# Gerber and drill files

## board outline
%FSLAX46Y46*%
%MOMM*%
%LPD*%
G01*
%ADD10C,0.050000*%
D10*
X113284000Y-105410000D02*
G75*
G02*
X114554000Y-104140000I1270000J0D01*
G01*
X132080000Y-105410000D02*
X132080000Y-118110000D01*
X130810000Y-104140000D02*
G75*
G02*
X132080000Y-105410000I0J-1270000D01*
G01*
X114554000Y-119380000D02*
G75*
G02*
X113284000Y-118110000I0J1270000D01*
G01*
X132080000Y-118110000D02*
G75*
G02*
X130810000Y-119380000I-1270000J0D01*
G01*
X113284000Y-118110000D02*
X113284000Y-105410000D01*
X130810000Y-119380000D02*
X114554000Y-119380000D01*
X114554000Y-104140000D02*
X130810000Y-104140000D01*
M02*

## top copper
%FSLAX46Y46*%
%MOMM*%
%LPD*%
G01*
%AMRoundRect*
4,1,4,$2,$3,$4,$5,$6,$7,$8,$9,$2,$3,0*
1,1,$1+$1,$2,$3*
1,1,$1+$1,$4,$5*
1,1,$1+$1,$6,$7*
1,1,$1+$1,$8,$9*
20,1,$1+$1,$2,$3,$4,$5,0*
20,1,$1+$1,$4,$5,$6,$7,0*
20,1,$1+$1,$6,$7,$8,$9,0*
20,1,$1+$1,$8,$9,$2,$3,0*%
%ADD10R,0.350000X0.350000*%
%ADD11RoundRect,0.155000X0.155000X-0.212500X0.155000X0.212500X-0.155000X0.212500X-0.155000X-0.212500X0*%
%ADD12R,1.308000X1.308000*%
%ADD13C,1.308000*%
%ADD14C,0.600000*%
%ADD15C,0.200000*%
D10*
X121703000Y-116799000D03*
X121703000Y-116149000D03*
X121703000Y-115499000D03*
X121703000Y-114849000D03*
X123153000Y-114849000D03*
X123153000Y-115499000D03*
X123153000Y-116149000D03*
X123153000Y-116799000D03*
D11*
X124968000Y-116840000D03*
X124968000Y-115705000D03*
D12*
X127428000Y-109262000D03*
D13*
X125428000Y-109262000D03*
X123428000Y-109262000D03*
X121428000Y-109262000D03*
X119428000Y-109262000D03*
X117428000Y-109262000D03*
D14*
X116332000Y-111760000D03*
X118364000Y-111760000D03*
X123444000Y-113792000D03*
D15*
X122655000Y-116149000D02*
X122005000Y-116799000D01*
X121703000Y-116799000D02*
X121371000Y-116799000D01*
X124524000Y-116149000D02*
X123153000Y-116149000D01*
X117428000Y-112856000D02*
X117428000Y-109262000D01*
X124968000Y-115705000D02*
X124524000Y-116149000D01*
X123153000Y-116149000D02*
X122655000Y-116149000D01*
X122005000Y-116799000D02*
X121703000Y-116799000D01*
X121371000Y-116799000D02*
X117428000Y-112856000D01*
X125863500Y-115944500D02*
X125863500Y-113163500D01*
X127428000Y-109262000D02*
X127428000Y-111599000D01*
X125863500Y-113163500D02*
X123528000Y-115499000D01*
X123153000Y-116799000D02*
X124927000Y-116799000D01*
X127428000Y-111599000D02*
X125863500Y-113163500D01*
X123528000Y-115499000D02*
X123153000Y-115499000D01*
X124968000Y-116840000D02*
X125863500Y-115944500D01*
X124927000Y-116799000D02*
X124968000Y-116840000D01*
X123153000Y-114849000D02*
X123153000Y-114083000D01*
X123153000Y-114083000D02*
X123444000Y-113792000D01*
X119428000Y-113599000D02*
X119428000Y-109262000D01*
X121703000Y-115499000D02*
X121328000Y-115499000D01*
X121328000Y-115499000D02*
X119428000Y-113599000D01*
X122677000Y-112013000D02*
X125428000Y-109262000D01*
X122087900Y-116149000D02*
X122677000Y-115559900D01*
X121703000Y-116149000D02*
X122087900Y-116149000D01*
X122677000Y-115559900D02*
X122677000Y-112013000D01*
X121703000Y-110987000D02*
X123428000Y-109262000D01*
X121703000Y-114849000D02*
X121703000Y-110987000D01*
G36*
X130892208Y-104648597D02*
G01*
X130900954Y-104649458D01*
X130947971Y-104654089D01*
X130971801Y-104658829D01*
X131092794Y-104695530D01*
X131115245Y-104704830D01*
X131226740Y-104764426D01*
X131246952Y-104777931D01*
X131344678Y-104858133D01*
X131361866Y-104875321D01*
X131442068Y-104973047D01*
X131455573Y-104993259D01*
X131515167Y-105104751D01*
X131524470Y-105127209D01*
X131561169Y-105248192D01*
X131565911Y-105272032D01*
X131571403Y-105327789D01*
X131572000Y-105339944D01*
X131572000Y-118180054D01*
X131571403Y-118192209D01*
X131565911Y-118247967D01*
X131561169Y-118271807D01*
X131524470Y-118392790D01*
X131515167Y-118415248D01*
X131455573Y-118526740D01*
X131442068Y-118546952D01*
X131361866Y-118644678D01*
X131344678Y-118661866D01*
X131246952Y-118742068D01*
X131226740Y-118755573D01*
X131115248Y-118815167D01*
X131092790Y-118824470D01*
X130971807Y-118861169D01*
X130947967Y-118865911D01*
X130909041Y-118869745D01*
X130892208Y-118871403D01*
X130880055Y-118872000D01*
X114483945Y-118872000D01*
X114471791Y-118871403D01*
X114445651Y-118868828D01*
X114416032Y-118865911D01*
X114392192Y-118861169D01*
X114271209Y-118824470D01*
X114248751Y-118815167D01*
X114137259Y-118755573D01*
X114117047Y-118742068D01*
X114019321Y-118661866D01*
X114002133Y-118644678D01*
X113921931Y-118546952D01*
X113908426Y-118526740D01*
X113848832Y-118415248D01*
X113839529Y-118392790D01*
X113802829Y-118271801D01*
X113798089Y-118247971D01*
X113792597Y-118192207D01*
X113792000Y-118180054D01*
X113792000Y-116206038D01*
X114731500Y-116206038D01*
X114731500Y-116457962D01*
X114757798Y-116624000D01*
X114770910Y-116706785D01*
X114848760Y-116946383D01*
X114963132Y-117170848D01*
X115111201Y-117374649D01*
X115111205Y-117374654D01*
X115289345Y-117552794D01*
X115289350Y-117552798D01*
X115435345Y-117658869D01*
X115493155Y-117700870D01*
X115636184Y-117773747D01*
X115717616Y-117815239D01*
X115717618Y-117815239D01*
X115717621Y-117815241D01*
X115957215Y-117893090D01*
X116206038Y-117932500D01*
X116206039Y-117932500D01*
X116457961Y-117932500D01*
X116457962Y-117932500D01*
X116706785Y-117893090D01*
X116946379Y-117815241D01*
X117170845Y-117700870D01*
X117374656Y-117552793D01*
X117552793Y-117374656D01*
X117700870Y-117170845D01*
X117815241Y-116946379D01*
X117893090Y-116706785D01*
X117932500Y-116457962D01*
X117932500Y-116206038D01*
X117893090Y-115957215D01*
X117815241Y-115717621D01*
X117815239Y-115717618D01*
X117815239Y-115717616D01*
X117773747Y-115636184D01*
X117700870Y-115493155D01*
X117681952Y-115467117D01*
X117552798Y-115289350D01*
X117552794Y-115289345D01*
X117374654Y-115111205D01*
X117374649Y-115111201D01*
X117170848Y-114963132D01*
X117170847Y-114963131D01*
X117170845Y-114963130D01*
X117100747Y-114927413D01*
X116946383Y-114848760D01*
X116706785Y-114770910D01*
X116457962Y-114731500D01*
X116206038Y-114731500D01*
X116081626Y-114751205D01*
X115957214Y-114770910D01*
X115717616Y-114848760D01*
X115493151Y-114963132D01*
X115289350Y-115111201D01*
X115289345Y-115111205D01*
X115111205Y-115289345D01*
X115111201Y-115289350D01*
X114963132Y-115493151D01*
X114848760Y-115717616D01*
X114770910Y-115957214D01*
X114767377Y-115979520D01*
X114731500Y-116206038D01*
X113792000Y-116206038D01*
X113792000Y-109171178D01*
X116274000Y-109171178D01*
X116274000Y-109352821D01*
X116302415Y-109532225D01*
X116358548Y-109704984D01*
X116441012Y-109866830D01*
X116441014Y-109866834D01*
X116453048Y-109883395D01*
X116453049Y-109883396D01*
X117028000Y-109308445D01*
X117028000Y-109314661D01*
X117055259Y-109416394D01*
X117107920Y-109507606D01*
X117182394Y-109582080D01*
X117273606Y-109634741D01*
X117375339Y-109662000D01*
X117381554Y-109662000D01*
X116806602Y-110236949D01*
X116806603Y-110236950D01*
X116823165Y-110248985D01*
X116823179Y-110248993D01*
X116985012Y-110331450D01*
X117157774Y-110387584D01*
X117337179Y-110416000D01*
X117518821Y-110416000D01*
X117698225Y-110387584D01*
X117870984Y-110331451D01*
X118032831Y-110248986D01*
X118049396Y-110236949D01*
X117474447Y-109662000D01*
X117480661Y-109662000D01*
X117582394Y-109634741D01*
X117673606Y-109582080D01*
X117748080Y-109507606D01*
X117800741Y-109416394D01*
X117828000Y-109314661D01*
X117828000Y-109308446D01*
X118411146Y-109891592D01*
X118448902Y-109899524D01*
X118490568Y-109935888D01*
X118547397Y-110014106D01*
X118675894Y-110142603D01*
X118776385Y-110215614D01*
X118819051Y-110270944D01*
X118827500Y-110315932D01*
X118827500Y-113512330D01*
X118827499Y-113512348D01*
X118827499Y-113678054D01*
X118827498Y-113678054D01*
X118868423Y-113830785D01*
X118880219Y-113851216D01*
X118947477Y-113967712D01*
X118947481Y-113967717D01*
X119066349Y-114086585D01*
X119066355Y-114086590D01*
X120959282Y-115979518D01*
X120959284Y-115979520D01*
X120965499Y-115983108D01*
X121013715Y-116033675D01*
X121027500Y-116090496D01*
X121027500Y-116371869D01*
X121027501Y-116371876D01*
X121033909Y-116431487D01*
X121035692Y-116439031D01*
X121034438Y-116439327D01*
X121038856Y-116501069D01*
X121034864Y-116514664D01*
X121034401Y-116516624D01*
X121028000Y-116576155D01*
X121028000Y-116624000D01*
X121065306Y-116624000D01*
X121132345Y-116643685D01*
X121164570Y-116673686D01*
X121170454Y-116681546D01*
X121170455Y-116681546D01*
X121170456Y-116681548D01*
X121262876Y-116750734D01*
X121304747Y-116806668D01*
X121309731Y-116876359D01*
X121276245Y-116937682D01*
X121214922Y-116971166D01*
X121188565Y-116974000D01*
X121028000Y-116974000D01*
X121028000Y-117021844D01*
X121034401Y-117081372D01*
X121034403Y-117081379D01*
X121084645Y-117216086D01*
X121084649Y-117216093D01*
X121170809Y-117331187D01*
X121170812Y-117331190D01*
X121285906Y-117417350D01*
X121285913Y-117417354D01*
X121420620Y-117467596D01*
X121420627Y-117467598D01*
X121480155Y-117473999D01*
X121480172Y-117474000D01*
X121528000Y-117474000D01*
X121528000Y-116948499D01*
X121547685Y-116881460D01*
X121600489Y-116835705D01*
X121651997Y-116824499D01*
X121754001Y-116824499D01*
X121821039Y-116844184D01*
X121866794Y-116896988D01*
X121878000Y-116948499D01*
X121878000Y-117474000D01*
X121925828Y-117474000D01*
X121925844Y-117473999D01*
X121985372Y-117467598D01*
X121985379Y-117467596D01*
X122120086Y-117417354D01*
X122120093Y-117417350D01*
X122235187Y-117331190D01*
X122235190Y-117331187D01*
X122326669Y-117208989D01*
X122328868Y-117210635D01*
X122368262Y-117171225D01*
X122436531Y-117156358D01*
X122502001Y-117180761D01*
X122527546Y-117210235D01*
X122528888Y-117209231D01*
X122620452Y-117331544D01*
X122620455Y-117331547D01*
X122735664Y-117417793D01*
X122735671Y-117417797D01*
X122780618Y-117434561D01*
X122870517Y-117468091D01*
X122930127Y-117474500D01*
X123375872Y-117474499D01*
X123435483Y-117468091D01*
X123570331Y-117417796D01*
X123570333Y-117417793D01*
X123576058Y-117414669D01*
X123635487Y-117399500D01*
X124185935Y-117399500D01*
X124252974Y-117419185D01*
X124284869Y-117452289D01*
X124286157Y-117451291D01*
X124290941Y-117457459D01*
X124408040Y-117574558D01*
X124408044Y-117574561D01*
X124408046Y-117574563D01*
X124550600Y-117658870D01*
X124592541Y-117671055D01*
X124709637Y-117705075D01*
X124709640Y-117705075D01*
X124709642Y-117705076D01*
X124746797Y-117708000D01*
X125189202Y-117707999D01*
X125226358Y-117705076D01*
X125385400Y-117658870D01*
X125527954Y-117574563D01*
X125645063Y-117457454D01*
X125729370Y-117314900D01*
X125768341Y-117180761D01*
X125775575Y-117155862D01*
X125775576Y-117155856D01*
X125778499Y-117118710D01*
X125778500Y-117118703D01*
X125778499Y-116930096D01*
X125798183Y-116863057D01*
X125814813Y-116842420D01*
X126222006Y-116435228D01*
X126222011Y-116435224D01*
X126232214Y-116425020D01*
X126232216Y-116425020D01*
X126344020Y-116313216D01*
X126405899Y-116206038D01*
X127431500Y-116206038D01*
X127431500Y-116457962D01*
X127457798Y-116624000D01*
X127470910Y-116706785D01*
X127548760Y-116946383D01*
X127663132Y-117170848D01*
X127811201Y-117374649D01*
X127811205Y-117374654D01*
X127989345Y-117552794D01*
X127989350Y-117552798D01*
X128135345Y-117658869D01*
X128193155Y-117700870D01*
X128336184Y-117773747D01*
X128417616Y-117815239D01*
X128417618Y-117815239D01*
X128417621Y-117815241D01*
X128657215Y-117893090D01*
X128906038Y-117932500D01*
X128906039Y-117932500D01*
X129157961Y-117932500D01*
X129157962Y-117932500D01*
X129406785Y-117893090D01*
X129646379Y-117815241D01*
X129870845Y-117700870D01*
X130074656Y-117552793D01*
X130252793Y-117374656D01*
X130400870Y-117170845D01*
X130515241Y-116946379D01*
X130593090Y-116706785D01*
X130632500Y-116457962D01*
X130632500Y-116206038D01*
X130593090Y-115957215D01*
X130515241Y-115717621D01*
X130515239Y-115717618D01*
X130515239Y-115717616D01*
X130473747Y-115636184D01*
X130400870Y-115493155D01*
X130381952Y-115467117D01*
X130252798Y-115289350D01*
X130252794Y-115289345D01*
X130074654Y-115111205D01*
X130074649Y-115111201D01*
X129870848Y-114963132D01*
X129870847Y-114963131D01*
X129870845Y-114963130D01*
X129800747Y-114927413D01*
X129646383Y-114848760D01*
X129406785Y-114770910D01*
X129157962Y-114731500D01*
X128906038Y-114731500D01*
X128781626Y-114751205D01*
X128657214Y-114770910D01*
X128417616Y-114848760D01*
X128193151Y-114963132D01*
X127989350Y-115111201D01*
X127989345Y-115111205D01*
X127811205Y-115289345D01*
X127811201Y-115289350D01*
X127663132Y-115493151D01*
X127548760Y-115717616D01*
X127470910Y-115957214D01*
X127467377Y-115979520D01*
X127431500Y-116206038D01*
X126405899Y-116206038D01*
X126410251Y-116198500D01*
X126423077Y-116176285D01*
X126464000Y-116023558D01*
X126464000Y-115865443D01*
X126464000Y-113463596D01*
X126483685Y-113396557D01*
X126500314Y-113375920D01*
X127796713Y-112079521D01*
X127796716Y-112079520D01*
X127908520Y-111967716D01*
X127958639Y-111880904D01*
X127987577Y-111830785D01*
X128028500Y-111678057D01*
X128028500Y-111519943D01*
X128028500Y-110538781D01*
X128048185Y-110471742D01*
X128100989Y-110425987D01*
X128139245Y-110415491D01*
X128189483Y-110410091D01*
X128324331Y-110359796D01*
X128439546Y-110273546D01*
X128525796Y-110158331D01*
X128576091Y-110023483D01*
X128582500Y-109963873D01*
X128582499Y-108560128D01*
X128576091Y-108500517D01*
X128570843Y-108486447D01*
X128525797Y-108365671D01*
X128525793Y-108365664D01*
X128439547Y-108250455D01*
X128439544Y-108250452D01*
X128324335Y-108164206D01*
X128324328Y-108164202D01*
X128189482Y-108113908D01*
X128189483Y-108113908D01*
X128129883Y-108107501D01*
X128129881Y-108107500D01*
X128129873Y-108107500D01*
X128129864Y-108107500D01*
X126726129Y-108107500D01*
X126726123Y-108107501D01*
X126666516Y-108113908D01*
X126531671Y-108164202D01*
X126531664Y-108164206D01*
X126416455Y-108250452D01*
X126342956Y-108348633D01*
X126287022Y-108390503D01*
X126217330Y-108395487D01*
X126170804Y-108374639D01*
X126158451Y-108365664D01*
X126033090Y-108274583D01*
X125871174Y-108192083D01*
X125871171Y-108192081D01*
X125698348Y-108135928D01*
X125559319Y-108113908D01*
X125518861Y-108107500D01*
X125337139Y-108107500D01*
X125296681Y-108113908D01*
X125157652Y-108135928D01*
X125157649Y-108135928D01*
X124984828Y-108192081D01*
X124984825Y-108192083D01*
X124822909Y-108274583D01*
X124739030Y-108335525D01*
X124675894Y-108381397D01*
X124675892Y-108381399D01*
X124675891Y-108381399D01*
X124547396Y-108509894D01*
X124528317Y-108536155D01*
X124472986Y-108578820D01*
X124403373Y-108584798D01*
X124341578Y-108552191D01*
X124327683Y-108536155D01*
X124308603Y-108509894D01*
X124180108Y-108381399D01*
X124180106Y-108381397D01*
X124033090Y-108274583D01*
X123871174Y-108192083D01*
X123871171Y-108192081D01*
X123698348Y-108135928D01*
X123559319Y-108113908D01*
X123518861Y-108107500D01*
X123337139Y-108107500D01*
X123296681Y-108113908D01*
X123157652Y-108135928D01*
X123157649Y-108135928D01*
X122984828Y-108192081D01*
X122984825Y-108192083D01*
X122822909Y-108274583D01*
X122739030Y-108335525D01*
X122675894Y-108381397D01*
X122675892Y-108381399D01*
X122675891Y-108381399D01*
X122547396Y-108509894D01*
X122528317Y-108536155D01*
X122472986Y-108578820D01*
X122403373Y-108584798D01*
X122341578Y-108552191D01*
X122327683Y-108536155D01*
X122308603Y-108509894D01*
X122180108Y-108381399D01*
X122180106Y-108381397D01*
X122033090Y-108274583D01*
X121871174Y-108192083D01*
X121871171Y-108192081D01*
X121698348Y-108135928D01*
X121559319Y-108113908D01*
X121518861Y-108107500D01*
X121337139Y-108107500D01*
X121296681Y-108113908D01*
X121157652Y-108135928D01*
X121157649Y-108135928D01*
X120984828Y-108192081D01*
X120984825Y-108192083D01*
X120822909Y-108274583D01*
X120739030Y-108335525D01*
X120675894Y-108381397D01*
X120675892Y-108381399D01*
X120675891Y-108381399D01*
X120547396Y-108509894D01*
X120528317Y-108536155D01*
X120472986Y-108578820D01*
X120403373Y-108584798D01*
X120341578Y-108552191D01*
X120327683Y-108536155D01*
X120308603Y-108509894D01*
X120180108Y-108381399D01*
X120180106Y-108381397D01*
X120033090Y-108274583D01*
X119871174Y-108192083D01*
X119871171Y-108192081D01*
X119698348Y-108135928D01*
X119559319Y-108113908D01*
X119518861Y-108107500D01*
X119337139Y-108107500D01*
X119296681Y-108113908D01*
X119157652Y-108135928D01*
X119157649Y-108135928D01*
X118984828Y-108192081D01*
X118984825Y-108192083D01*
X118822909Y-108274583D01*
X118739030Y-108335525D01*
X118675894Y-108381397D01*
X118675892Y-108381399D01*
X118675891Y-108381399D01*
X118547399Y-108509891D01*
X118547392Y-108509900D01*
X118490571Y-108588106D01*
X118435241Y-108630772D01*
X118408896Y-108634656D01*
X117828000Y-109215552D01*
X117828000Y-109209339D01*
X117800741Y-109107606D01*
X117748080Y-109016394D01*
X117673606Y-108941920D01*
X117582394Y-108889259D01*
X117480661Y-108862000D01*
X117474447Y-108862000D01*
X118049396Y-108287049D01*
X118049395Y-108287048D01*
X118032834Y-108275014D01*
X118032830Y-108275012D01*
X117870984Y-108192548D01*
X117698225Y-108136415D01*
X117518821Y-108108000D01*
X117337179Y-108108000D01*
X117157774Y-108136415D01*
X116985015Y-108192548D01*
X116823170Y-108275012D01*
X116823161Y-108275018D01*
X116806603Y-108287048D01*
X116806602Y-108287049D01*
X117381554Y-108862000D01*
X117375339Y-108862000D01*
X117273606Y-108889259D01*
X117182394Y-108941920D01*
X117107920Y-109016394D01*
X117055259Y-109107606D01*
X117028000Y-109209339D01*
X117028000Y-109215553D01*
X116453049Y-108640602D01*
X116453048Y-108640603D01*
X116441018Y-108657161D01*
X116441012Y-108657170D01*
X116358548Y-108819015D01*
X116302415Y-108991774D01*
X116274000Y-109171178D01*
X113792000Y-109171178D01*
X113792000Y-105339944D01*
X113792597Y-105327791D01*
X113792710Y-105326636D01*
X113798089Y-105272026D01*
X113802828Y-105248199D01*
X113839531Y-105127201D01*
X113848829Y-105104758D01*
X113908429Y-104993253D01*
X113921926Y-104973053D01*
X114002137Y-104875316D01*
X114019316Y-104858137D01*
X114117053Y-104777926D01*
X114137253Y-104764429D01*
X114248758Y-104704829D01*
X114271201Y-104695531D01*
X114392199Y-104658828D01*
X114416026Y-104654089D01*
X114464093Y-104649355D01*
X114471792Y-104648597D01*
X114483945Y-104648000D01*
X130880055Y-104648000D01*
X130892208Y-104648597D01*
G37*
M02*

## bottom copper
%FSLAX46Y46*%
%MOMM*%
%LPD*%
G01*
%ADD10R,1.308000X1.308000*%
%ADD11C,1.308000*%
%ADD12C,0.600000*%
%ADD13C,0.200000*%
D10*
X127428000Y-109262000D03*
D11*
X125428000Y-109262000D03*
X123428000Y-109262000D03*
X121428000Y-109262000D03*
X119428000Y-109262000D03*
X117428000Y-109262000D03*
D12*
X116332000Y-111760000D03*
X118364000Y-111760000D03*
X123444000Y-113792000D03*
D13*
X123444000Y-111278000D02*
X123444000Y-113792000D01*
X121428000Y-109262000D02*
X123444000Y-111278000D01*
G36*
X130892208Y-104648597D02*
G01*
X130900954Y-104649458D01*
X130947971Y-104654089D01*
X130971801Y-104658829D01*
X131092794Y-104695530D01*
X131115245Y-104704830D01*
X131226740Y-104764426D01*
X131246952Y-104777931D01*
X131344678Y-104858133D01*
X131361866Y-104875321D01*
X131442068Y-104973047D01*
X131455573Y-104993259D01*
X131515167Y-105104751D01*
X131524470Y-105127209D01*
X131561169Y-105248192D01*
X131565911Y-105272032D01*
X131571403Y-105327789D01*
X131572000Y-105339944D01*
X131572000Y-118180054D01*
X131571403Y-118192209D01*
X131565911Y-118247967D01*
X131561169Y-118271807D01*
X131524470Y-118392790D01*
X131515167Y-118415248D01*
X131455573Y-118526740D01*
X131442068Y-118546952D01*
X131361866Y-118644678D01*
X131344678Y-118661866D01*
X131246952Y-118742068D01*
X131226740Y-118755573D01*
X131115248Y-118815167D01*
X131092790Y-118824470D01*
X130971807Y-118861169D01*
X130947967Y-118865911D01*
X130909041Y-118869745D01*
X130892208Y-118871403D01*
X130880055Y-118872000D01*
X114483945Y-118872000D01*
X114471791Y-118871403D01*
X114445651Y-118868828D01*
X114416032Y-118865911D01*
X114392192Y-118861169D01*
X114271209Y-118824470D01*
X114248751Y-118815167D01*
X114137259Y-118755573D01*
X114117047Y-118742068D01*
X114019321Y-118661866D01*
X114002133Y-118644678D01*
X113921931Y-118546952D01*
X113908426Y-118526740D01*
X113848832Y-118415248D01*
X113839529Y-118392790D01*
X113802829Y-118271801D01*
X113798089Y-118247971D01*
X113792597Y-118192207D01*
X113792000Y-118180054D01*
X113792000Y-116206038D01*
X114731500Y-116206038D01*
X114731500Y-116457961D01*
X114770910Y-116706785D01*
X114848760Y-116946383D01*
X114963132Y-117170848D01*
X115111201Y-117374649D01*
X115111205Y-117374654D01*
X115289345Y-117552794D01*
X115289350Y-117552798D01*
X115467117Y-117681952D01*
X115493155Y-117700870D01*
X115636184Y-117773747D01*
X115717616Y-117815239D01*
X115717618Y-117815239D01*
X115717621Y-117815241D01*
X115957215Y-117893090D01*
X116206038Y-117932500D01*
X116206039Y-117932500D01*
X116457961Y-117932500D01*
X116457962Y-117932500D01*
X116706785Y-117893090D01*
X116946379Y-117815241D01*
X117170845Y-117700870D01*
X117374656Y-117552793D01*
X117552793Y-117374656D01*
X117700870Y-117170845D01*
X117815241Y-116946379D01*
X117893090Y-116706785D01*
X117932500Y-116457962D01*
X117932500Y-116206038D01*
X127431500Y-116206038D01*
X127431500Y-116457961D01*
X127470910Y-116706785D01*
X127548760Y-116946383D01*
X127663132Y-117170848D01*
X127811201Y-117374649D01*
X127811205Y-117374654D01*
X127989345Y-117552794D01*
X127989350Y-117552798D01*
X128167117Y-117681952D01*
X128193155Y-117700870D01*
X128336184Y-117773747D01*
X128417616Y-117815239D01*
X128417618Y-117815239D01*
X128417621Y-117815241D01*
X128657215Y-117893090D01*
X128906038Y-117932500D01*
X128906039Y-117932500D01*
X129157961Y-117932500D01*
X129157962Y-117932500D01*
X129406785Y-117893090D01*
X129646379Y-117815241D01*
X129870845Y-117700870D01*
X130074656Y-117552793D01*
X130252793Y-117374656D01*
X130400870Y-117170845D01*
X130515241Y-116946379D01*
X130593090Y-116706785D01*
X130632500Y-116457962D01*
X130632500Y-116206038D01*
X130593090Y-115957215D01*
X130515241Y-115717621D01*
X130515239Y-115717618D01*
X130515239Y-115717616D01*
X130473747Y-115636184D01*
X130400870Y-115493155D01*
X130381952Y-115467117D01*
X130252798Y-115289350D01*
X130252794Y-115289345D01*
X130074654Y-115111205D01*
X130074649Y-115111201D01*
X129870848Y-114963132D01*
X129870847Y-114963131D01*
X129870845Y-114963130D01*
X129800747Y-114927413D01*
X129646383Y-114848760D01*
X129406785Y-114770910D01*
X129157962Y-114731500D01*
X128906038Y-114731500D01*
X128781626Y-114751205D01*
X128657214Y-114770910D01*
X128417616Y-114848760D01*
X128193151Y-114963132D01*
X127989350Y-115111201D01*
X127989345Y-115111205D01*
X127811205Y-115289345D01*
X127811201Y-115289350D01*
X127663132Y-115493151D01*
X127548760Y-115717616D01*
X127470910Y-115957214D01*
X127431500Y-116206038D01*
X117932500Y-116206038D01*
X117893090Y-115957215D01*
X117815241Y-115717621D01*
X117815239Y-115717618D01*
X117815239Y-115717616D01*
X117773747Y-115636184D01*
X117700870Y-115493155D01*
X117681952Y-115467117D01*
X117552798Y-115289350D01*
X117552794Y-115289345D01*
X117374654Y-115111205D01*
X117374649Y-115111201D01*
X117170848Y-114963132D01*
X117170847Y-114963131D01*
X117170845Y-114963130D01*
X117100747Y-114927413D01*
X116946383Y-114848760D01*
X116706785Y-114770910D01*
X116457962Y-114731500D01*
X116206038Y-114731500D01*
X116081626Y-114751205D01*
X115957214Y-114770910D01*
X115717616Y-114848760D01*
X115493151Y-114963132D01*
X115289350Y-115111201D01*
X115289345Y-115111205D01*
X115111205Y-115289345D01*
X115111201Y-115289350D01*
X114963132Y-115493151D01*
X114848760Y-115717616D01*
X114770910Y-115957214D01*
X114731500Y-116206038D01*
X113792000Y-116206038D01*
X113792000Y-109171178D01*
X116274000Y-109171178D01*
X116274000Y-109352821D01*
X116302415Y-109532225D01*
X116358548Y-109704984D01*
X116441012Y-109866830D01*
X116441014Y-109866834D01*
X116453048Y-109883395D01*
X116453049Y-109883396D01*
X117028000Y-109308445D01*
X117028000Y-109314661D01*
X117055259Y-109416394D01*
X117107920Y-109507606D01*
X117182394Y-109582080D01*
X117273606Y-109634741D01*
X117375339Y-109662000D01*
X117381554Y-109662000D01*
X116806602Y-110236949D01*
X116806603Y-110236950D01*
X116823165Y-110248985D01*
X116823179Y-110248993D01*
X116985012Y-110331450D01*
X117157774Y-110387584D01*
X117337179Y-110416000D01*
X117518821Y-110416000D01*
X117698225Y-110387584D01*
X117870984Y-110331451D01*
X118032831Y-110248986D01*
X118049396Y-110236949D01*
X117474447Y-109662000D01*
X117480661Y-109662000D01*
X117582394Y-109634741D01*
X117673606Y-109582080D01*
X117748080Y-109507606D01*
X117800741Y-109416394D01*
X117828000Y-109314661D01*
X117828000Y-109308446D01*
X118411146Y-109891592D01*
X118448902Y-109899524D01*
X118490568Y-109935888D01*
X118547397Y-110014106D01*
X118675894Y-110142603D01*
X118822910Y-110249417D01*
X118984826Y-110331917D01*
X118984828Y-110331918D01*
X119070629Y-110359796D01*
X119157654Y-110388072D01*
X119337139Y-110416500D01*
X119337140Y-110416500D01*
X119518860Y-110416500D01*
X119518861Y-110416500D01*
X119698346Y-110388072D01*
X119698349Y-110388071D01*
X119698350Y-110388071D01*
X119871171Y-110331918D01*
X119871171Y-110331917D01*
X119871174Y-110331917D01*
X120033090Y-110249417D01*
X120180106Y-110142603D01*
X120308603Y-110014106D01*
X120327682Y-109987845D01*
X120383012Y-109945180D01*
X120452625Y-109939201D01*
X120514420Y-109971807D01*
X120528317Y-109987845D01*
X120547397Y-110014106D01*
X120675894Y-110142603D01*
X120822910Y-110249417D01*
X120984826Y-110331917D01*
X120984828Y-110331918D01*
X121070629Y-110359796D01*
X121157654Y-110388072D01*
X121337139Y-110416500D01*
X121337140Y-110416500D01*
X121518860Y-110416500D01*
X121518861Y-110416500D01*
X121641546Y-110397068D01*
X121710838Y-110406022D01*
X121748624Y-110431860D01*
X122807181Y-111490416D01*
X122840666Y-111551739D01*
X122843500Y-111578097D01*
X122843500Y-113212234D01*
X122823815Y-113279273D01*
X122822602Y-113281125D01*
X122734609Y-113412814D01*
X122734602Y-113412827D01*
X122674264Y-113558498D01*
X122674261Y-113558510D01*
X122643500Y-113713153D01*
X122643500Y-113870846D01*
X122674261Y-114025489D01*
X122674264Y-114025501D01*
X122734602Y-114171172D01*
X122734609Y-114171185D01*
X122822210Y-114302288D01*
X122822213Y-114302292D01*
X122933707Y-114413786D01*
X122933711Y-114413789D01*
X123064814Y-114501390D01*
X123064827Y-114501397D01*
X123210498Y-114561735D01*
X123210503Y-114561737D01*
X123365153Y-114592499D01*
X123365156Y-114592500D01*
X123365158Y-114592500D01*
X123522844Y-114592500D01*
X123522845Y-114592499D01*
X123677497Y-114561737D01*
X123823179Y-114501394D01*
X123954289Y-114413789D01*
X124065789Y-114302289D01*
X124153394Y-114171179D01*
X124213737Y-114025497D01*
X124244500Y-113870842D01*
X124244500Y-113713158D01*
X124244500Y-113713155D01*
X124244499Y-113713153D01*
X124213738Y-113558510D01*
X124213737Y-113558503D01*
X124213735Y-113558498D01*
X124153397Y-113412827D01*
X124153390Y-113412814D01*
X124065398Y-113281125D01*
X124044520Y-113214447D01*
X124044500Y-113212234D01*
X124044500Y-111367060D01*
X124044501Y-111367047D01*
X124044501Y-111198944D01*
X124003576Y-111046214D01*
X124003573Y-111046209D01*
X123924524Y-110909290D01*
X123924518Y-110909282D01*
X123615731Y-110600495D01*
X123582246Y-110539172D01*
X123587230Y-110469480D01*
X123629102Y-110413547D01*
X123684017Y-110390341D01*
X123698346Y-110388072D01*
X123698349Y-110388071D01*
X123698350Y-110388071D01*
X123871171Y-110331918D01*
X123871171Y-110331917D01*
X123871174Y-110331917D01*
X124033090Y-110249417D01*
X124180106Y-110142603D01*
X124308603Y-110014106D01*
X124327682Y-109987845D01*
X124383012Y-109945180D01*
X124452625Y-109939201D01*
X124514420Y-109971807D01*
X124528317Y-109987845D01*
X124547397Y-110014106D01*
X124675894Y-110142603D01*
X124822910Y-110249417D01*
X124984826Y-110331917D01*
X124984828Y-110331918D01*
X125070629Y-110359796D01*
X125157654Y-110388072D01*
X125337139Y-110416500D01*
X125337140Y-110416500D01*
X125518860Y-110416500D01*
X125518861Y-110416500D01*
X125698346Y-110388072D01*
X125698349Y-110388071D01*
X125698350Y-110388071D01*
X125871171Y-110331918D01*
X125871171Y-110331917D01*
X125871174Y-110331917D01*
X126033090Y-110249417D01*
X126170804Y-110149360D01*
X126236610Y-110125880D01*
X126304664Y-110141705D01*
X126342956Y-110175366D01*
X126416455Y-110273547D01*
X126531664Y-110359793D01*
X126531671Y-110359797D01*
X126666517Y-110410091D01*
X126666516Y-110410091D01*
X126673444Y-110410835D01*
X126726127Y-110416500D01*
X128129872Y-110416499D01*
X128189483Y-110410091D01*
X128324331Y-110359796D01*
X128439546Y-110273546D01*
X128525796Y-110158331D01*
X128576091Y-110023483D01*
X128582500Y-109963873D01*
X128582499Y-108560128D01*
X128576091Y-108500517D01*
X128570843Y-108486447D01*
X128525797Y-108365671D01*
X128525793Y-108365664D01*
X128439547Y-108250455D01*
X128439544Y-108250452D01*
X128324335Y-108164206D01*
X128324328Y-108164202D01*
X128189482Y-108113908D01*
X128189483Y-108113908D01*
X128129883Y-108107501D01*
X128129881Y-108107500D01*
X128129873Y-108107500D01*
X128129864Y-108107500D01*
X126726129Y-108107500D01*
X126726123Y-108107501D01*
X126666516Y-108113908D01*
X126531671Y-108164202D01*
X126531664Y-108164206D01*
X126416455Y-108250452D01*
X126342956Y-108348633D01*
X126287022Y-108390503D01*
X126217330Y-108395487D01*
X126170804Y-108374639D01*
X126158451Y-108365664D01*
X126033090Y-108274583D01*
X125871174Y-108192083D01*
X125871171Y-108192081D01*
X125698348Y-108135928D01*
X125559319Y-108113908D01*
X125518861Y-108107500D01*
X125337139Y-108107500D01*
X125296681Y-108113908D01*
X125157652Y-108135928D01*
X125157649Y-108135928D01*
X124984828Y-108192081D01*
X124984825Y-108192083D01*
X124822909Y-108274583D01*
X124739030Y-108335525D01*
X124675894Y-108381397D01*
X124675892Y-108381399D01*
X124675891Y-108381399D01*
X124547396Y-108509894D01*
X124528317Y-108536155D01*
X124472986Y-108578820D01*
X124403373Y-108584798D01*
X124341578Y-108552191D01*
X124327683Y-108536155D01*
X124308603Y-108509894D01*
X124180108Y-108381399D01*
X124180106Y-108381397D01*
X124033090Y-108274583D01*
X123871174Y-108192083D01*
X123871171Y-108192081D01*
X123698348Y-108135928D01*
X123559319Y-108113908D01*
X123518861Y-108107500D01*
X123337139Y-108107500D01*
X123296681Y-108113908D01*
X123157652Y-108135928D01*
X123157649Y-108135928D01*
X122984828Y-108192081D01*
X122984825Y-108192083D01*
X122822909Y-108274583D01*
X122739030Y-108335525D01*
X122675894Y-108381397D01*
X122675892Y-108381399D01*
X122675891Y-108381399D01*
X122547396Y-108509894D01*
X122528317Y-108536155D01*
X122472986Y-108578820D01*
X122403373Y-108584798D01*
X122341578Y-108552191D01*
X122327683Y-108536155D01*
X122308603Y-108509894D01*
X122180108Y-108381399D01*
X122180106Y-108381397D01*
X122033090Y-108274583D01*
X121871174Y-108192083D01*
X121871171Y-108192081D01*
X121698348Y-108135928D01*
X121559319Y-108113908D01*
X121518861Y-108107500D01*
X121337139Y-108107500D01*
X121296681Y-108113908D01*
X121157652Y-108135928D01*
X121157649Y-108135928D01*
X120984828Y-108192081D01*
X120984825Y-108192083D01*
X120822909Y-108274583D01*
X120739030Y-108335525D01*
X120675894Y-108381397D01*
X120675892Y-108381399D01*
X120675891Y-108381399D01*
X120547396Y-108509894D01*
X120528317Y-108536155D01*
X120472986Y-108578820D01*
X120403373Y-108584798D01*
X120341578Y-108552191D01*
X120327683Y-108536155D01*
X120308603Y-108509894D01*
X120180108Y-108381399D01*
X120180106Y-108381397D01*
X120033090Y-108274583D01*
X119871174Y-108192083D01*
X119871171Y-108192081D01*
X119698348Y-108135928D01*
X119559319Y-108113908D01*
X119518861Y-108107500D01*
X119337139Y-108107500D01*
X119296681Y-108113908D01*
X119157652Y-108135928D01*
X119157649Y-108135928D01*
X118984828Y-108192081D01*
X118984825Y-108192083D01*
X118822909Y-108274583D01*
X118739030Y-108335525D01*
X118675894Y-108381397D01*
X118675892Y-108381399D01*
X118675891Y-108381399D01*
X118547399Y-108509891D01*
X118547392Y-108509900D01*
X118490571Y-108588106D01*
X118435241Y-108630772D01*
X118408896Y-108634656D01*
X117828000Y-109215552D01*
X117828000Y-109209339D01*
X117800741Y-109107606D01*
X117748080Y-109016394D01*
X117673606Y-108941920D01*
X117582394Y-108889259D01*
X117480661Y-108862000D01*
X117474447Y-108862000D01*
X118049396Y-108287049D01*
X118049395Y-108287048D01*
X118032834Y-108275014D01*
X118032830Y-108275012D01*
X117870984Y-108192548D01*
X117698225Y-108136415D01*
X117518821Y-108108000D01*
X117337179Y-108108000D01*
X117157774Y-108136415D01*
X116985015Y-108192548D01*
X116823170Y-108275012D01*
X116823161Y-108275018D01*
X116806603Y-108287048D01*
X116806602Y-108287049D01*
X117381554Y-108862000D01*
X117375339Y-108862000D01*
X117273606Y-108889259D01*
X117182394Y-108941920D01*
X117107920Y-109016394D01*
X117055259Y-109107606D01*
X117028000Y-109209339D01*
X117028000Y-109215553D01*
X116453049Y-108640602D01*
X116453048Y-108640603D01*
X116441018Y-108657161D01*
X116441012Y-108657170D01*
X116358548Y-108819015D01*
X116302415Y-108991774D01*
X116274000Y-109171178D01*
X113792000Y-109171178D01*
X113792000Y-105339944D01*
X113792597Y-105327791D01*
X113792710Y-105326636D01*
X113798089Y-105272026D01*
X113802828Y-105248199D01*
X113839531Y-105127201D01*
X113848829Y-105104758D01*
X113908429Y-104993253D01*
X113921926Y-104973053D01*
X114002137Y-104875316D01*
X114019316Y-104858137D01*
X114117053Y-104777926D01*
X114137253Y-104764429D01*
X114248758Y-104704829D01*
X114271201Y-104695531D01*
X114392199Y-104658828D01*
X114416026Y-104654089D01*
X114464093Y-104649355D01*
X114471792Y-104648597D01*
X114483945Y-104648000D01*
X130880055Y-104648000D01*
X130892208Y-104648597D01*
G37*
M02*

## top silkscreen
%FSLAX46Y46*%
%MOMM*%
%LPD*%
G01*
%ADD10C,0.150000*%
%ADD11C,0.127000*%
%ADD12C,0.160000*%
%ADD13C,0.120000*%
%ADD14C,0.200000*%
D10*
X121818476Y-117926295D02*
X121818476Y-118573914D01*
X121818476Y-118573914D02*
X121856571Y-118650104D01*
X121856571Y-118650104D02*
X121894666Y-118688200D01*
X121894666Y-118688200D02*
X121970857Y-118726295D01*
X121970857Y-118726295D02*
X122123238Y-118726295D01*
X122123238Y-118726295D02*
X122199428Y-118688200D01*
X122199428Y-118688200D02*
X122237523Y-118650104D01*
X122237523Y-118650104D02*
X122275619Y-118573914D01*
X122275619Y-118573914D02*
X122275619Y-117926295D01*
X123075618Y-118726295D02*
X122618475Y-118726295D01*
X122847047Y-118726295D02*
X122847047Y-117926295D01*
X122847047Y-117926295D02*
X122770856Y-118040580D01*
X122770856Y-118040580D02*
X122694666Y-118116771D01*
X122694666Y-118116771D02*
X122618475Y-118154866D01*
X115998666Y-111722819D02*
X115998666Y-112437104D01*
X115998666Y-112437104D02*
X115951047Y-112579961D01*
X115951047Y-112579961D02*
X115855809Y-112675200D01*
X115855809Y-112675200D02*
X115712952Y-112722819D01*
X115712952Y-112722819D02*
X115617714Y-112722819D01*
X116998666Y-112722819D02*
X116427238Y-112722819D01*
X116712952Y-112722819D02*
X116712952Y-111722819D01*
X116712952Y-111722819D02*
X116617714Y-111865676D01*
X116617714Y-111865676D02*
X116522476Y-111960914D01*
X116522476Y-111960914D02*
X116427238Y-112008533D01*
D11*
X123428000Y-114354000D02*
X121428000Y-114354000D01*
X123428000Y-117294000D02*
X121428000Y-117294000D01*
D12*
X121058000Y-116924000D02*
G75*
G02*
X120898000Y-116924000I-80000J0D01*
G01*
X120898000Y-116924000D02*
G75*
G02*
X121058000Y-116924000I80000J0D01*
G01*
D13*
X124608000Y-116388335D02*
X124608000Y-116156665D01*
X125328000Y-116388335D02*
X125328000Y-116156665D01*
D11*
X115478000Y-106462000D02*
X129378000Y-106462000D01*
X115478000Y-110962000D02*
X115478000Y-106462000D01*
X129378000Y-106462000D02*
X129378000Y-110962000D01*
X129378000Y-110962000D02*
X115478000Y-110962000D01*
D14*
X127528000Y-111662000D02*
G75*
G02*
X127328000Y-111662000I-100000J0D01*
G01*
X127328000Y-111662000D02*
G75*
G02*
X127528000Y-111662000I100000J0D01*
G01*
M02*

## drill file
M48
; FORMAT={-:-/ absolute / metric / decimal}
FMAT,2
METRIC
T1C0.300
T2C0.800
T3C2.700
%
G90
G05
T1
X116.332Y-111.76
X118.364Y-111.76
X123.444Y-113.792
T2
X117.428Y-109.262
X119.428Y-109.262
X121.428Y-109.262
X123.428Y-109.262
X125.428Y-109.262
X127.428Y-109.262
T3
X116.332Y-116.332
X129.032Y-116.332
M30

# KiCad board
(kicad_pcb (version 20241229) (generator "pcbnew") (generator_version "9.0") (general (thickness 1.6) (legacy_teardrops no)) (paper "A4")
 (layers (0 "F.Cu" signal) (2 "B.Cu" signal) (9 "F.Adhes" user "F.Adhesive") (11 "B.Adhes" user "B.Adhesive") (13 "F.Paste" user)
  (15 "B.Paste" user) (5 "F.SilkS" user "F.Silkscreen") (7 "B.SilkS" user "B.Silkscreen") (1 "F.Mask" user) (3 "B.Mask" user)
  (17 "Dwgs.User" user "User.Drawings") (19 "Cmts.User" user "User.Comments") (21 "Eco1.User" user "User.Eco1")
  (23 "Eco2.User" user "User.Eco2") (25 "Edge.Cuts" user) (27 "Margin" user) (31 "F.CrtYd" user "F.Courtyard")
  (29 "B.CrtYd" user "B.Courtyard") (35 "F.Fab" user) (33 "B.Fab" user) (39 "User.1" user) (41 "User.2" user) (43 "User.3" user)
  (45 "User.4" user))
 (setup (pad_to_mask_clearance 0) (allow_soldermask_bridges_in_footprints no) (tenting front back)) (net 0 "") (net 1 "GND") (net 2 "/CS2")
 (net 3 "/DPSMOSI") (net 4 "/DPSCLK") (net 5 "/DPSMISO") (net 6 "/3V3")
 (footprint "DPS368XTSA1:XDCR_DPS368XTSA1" (layer "F.Cu") (at 122.428 115.824 180)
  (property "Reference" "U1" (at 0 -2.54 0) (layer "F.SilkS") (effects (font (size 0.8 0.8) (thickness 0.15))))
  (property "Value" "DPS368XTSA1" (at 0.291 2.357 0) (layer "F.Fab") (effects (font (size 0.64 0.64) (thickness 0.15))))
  (fp_line (start -1 1.47) (end 1 1.47) (stroke (width 0.127) (type solid)) (layer "F.SilkS"))
  (fp_line (start -1 -1.47) (end 1 -1.47) (stroke (width 0.127) (type solid)) (layer "F.SilkS"))
  (fp_circle (center 1.45 -1.1) (end 1.53 -1.1) (stroke (width 0.16) (type solid)) (fill no) (layer "F.SilkS"))
  (pad "1" smd rect (at 0.725 -0.975 180) (size 0.35 0.35) (layers "F.Cu" "F.Mask") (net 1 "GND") (solder_mask_margin 0.102))
  (pad "2" smd rect (at 0.725 -0.325 180) (size 0.35 0.35) (layers "F.Cu" "F.Mask") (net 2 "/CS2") (solder_mask_margin 0.102))
  (pad "3" smd rect (at 0.725 0.325 180) (size 0.35 0.35) (layers "F.Cu" "F.Mask") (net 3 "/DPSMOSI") (solder_mask_margin 0.102))
  (pad "4" smd rect (at 0.725 0.975 180) (size 0.35 0.35) (layers "F.Cu" "F.Mask") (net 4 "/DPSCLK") (solder_mask_margin 0.102))
  (pad "5" smd rect (at -0.725 0.975 180) (size 0.35 0.35) (layers "F.Cu" "F.Mask") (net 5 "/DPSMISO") (solder_mask_margin 0.102))
  (pad "6" smd rect (at -0.725 0.325 180) (size 0.35 0.35) (layers "F.Cu" "F.Mask") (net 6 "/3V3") (solder_mask_margin 0.102))
  (pad "7" smd rect (at -0.725 -0.325 180) (size 0.35 0.35) (layers "F.Cu" "F.Mask") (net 1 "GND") (solder_mask_margin 0.102))
  (pad "8" smd rect (at -0.725 -0.975 180) (size 0.35 0.35) (layers "F.Cu" "F.Mask") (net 6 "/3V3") (solder_mask_margin 0.102)))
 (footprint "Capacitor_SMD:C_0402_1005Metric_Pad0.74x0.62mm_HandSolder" (layer "F.Cu") (at 124.968 116.2725 90)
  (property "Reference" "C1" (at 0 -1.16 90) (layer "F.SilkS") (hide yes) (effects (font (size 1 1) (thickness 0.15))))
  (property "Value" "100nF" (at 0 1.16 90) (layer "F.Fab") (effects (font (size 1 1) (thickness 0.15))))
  (fp_line (start -0.115835 -0.36) (end 0.115835 -0.36) (stroke (width 0.12) (type solid)) (layer "F.SilkS"))
  (fp_line (start -0.115835 0.36) (end 0.115835 0.36) (stroke (width 0.12) (type solid)) (layer "F.SilkS"))
  (pad "1" smd roundrect (at -0.5675 0 90) (size 0.735 0.62) (layers "F.Cu" "F.Mask" "F.Paste") (roundrect_rratio 0.25) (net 6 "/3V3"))
  (pad "2" smd roundrect (at 0.5675 0 90) (size 0.735 0.62) (layers "F.Cu" "F.Mask" "F.Paste") (roundrect_rratio 0.25) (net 1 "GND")))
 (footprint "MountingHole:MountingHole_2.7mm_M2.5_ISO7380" (layer "F.Cu") (at 116.332 116.332)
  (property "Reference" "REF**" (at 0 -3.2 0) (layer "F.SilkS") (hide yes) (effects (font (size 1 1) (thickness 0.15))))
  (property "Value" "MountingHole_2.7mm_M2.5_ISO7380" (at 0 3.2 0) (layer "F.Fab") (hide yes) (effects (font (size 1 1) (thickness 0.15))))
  (pad "" np_thru_hole circle (at 0 0) (size 2.7 2.7) (drill 2.7) (layers "*.Cu" "*.Mask")))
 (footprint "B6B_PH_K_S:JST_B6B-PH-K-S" (layer "F.Cu") (at 122.428 108.712)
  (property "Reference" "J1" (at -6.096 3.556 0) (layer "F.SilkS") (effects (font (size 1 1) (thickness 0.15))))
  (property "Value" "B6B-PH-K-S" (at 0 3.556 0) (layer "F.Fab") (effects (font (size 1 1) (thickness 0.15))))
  (fp_line (start -6.95 -2.25) (end 6.95 -2.25) (stroke (width 0.127) (type solid)) (layer "F.SilkS"))
  (fp_line (start -6.95 2.25) (end -6.95 -2.25) (stroke (width 0.127) (type solid)) (layer "F.SilkS"))
  (fp_line (start 6.95 -2.25) (end 6.95 2.25) (stroke (width 0.127) (type solid)) (layer "F.SilkS"))
  (fp_line (start 6.95 2.25) (end -6.95 2.25) (stroke (width 0.127) (type solid)) (layer "F.SilkS"))
  (fp_circle (center 5 2.95) (end 5.1 2.95) (stroke (width 0.2) (type solid)) (fill no) (layer "F.SilkS"))
  (pad "1" thru_hole rect (at 5 0.55) (size 1.308 1.308) (drill 0.8) (layers "*.Cu" "*.Mask") (remove_unused_layers no) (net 6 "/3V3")
   (solder_mask_margin 0.102))
  (pad "2" thru_hole circle (at 3 0.55) (size 1.308 1.308) (drill 0.8) (layers "*.Cu" "*.Mask") (remove_unused_layers no) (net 2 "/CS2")
   (solder_mask_margin 0.102))
  (pad "3" thru_hole circle (at 1 0.55) (size 1.308 1.308) (drill 0.8) (layers "*.Cu" "*.Mask") (remove_unused_layers no) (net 4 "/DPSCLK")
   (solder_mask_margin 0.102))
  (pad "4" thru_hole circle (at -1 0.55) (size 1.308 1.308) (drill 0.8) (layers "*.Cu" "*.Mask") (remove_unused_layers no)
   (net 5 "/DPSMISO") (solder_mask_margin 0.102))
  (pad "5" thru_hole circle (at -3 0.55) (size 1.308 1.308) (drill 0.8) (layers "*.Cu" "*.Mask") (remove_unused_layers no)
   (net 3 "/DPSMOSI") (solder_mask_margin 0.102))
  (pad "6" thru_hole circle (at -5 0.55) (size 1.308 1.308) (drill 0.8) (layers "*.Cu" "*.Mask") (remove_unused_layers no) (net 1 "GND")
   (solder_mask_margin 0.102)))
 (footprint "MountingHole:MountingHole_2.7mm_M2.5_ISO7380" (layer "F.Cu") (at 129.032 116.332)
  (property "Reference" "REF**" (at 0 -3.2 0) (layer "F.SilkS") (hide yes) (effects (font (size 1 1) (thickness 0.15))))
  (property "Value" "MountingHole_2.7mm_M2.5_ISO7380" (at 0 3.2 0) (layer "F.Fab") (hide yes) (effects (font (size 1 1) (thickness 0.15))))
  (pad "" np_thru_hole circle (at 0 0) (size 2.7 2.7) (drill 2.7) (layers "*.Cu" "*.Mask")))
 (gr_arc (start 113.284 105.41) (mid 113.655974 104.511974) (end 114.554 104.14) (stroke (width 0.05) (type default)) (layer "Edge.Cuts"))
 (gr_line (start 132.08 105.41) (end 132.08 118.11) (stroke (width 0.05) (type default)) (layer "Edge.Cuts"))
 (gr_arc (start 130.81 104.14) (mid 131.708026 104.511974) (end 132.08 105.41) (stroke (width 0.05) (type default)) (layer "Edge.Cuts"))
 (gr_arc (start 114.554 119.38) (mid 113.655974 119.008026) (end 113.284 118.11) (stroke (width 0.05) (type default)) (layer "Edge.Cuts"))
 (gr_arc (start 132.08 118.11) (mid 131.708026 119.008026) (end 130.81 119.38) (stroke (width 0.05) (type default)) (layer "Edge.Cuts"))
 (gr_line (start 113.284 118.11) (end 113.284 105.41) (stroke (width 0.05) (type default)) (layer "Edge.Cuts"))
 (gr_line (start 130.81 119.38) (end 114.554 119.38) (stroke (width 0.05) (type default)) (layer "Edge.Cuts"))
 (gr_line (start 114.554 104.14) (end 130.81 104.14) (stroke (width 0.05) (type default)) (layer "Edge.Cuts"))
 (segment (start 122.655 116.149) (end 122.005 116.799) (width 0.2) (layer "F.Cu") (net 1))
 (segment (start 121.703 116.799) (end 121.371 116.799) (width 0.2) (layer "F.Cu") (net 1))
 (segment (start 124.524 116.149) (end 123.153 116.149) (width 0.2) (layer "F.Cu") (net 1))
 (segment (start 117.428 112.856) (end 117.428 109.262) (width 0.2) (layer "F.Cu") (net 1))
 (segment (start 124.968 115.705) (end 124.524 116.149) (width 0.2) (layer "F.Cu") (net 1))
 (segment (start 123.153 116.149) (end 122.655 116.149) (width 0.2) (layer "F.Cu") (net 1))
 (segment (start 122.005 116.799) (end 121.703 116.799) (width 0.2) (layer "F.Cu") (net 1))
 (segment (start 121.371 116.799) (end 117.428 112.856) (width 0.2) (layer "F.Cu") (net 1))
 (via (at 116.332 111.76) (size 0.6) (drill 0.3) (layers "F.Cu" "B.Cu") (free yes) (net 1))
 (via (at 118.364 111.76) (size 0.6) (drill 0.3) (layers "F.Cu" "B.Cu") (free yes) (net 1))
 (segment (start 125.8635 115.9445) (end 125.8635 113.1635) (width 0.2) (layer "F.Cu") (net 6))
 (segment (start 127.428 109.262) (end 127.428 111.599) (width 0.2) (layer "F.Cu") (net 6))
 (segment (start 125.8635 113.1635) (end 123.528 115.499) (width 0.2) (layer "F.Cu") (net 6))
 (segment (start 123.153 116.799) (end 124.927 116.799) (width 0.2) (layer "F.Cu") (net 6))
 (segment (start 127.428 111.599) (end 125.8635 113.1635) (width 0.2) (layer "F.Cu") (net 6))
 (segment (start 123.528 115.499) (end 123.153 115.499) (width 0.2) (layer "F.Cu") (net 6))
 (segment (start 124.968 116.84) (end 125.8635 115.9445) (width 0.2) (layer "F.Cu") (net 6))
 (segment (start 124.927 116.799) (end 124.968 116.84) (width 0.2) (layer "F.Cu") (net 6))
 (segment (start 123.153 114.849) (end 123.153 114.083) (width 0.2) (layer "F.Cu") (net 5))
 (segment (start 123.153 114.083) (end 123.444 113.792) (width 0.2) (layer "F.Cu") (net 5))
 (via (at 123.444 113.792) (size 0.6) (drill 0.3) (layers "F.Cu" "B.Cu") (free yes) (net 5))
 (segment (start 123.444 111.278) (end 123.444 113.792) (width 0.2) (layer "B.Cu") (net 5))
 (segment (start 121.428 109.262) (end 123.444 111.278) (width 0.2) (layer "B.Cu") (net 5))
 (segment (start 119.428 113.599) (end 119.428 109.262) (width 0.2) (layer "F.Cu") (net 3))
 (segment (start 121.703 115.499) (end 121.328 115.499) (width 0.2) (layer "F.Cu") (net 3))
 (segment (start 121.328 115.499) (end 119.428 113.599) (width 0.2) (layer "F.Cu") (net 3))
 (segment (start 122.677 112.013) (end 125.428 109.262) (width 0.2) (layer "F.Cu") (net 2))
 (segment (start 122.0879 116.149) (end 122.677 115.5599) (width 0.2) (layer "F.Cu") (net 2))
 (segment (start 121.703 116.149) (end 122.0879 116.149) (width 0.2) (layer "F.Cu") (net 2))
 (segment (start 122.677 115.5599) (end 122.677 112.013) (width 0.2) (layer "F.Cu") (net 2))
 (segment (start 121.703 110.987) (end 123.428 109.262) (width 0.2) (layer "F.Cu") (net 4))
 (segment (start 121.703 114.849) (end 121.703 110.987) (width 0.2) (layer "F.Cu") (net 4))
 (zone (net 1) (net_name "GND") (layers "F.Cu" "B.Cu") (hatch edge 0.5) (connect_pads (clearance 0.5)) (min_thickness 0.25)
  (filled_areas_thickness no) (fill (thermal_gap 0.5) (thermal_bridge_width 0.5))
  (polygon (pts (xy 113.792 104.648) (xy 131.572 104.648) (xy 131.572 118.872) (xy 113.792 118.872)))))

